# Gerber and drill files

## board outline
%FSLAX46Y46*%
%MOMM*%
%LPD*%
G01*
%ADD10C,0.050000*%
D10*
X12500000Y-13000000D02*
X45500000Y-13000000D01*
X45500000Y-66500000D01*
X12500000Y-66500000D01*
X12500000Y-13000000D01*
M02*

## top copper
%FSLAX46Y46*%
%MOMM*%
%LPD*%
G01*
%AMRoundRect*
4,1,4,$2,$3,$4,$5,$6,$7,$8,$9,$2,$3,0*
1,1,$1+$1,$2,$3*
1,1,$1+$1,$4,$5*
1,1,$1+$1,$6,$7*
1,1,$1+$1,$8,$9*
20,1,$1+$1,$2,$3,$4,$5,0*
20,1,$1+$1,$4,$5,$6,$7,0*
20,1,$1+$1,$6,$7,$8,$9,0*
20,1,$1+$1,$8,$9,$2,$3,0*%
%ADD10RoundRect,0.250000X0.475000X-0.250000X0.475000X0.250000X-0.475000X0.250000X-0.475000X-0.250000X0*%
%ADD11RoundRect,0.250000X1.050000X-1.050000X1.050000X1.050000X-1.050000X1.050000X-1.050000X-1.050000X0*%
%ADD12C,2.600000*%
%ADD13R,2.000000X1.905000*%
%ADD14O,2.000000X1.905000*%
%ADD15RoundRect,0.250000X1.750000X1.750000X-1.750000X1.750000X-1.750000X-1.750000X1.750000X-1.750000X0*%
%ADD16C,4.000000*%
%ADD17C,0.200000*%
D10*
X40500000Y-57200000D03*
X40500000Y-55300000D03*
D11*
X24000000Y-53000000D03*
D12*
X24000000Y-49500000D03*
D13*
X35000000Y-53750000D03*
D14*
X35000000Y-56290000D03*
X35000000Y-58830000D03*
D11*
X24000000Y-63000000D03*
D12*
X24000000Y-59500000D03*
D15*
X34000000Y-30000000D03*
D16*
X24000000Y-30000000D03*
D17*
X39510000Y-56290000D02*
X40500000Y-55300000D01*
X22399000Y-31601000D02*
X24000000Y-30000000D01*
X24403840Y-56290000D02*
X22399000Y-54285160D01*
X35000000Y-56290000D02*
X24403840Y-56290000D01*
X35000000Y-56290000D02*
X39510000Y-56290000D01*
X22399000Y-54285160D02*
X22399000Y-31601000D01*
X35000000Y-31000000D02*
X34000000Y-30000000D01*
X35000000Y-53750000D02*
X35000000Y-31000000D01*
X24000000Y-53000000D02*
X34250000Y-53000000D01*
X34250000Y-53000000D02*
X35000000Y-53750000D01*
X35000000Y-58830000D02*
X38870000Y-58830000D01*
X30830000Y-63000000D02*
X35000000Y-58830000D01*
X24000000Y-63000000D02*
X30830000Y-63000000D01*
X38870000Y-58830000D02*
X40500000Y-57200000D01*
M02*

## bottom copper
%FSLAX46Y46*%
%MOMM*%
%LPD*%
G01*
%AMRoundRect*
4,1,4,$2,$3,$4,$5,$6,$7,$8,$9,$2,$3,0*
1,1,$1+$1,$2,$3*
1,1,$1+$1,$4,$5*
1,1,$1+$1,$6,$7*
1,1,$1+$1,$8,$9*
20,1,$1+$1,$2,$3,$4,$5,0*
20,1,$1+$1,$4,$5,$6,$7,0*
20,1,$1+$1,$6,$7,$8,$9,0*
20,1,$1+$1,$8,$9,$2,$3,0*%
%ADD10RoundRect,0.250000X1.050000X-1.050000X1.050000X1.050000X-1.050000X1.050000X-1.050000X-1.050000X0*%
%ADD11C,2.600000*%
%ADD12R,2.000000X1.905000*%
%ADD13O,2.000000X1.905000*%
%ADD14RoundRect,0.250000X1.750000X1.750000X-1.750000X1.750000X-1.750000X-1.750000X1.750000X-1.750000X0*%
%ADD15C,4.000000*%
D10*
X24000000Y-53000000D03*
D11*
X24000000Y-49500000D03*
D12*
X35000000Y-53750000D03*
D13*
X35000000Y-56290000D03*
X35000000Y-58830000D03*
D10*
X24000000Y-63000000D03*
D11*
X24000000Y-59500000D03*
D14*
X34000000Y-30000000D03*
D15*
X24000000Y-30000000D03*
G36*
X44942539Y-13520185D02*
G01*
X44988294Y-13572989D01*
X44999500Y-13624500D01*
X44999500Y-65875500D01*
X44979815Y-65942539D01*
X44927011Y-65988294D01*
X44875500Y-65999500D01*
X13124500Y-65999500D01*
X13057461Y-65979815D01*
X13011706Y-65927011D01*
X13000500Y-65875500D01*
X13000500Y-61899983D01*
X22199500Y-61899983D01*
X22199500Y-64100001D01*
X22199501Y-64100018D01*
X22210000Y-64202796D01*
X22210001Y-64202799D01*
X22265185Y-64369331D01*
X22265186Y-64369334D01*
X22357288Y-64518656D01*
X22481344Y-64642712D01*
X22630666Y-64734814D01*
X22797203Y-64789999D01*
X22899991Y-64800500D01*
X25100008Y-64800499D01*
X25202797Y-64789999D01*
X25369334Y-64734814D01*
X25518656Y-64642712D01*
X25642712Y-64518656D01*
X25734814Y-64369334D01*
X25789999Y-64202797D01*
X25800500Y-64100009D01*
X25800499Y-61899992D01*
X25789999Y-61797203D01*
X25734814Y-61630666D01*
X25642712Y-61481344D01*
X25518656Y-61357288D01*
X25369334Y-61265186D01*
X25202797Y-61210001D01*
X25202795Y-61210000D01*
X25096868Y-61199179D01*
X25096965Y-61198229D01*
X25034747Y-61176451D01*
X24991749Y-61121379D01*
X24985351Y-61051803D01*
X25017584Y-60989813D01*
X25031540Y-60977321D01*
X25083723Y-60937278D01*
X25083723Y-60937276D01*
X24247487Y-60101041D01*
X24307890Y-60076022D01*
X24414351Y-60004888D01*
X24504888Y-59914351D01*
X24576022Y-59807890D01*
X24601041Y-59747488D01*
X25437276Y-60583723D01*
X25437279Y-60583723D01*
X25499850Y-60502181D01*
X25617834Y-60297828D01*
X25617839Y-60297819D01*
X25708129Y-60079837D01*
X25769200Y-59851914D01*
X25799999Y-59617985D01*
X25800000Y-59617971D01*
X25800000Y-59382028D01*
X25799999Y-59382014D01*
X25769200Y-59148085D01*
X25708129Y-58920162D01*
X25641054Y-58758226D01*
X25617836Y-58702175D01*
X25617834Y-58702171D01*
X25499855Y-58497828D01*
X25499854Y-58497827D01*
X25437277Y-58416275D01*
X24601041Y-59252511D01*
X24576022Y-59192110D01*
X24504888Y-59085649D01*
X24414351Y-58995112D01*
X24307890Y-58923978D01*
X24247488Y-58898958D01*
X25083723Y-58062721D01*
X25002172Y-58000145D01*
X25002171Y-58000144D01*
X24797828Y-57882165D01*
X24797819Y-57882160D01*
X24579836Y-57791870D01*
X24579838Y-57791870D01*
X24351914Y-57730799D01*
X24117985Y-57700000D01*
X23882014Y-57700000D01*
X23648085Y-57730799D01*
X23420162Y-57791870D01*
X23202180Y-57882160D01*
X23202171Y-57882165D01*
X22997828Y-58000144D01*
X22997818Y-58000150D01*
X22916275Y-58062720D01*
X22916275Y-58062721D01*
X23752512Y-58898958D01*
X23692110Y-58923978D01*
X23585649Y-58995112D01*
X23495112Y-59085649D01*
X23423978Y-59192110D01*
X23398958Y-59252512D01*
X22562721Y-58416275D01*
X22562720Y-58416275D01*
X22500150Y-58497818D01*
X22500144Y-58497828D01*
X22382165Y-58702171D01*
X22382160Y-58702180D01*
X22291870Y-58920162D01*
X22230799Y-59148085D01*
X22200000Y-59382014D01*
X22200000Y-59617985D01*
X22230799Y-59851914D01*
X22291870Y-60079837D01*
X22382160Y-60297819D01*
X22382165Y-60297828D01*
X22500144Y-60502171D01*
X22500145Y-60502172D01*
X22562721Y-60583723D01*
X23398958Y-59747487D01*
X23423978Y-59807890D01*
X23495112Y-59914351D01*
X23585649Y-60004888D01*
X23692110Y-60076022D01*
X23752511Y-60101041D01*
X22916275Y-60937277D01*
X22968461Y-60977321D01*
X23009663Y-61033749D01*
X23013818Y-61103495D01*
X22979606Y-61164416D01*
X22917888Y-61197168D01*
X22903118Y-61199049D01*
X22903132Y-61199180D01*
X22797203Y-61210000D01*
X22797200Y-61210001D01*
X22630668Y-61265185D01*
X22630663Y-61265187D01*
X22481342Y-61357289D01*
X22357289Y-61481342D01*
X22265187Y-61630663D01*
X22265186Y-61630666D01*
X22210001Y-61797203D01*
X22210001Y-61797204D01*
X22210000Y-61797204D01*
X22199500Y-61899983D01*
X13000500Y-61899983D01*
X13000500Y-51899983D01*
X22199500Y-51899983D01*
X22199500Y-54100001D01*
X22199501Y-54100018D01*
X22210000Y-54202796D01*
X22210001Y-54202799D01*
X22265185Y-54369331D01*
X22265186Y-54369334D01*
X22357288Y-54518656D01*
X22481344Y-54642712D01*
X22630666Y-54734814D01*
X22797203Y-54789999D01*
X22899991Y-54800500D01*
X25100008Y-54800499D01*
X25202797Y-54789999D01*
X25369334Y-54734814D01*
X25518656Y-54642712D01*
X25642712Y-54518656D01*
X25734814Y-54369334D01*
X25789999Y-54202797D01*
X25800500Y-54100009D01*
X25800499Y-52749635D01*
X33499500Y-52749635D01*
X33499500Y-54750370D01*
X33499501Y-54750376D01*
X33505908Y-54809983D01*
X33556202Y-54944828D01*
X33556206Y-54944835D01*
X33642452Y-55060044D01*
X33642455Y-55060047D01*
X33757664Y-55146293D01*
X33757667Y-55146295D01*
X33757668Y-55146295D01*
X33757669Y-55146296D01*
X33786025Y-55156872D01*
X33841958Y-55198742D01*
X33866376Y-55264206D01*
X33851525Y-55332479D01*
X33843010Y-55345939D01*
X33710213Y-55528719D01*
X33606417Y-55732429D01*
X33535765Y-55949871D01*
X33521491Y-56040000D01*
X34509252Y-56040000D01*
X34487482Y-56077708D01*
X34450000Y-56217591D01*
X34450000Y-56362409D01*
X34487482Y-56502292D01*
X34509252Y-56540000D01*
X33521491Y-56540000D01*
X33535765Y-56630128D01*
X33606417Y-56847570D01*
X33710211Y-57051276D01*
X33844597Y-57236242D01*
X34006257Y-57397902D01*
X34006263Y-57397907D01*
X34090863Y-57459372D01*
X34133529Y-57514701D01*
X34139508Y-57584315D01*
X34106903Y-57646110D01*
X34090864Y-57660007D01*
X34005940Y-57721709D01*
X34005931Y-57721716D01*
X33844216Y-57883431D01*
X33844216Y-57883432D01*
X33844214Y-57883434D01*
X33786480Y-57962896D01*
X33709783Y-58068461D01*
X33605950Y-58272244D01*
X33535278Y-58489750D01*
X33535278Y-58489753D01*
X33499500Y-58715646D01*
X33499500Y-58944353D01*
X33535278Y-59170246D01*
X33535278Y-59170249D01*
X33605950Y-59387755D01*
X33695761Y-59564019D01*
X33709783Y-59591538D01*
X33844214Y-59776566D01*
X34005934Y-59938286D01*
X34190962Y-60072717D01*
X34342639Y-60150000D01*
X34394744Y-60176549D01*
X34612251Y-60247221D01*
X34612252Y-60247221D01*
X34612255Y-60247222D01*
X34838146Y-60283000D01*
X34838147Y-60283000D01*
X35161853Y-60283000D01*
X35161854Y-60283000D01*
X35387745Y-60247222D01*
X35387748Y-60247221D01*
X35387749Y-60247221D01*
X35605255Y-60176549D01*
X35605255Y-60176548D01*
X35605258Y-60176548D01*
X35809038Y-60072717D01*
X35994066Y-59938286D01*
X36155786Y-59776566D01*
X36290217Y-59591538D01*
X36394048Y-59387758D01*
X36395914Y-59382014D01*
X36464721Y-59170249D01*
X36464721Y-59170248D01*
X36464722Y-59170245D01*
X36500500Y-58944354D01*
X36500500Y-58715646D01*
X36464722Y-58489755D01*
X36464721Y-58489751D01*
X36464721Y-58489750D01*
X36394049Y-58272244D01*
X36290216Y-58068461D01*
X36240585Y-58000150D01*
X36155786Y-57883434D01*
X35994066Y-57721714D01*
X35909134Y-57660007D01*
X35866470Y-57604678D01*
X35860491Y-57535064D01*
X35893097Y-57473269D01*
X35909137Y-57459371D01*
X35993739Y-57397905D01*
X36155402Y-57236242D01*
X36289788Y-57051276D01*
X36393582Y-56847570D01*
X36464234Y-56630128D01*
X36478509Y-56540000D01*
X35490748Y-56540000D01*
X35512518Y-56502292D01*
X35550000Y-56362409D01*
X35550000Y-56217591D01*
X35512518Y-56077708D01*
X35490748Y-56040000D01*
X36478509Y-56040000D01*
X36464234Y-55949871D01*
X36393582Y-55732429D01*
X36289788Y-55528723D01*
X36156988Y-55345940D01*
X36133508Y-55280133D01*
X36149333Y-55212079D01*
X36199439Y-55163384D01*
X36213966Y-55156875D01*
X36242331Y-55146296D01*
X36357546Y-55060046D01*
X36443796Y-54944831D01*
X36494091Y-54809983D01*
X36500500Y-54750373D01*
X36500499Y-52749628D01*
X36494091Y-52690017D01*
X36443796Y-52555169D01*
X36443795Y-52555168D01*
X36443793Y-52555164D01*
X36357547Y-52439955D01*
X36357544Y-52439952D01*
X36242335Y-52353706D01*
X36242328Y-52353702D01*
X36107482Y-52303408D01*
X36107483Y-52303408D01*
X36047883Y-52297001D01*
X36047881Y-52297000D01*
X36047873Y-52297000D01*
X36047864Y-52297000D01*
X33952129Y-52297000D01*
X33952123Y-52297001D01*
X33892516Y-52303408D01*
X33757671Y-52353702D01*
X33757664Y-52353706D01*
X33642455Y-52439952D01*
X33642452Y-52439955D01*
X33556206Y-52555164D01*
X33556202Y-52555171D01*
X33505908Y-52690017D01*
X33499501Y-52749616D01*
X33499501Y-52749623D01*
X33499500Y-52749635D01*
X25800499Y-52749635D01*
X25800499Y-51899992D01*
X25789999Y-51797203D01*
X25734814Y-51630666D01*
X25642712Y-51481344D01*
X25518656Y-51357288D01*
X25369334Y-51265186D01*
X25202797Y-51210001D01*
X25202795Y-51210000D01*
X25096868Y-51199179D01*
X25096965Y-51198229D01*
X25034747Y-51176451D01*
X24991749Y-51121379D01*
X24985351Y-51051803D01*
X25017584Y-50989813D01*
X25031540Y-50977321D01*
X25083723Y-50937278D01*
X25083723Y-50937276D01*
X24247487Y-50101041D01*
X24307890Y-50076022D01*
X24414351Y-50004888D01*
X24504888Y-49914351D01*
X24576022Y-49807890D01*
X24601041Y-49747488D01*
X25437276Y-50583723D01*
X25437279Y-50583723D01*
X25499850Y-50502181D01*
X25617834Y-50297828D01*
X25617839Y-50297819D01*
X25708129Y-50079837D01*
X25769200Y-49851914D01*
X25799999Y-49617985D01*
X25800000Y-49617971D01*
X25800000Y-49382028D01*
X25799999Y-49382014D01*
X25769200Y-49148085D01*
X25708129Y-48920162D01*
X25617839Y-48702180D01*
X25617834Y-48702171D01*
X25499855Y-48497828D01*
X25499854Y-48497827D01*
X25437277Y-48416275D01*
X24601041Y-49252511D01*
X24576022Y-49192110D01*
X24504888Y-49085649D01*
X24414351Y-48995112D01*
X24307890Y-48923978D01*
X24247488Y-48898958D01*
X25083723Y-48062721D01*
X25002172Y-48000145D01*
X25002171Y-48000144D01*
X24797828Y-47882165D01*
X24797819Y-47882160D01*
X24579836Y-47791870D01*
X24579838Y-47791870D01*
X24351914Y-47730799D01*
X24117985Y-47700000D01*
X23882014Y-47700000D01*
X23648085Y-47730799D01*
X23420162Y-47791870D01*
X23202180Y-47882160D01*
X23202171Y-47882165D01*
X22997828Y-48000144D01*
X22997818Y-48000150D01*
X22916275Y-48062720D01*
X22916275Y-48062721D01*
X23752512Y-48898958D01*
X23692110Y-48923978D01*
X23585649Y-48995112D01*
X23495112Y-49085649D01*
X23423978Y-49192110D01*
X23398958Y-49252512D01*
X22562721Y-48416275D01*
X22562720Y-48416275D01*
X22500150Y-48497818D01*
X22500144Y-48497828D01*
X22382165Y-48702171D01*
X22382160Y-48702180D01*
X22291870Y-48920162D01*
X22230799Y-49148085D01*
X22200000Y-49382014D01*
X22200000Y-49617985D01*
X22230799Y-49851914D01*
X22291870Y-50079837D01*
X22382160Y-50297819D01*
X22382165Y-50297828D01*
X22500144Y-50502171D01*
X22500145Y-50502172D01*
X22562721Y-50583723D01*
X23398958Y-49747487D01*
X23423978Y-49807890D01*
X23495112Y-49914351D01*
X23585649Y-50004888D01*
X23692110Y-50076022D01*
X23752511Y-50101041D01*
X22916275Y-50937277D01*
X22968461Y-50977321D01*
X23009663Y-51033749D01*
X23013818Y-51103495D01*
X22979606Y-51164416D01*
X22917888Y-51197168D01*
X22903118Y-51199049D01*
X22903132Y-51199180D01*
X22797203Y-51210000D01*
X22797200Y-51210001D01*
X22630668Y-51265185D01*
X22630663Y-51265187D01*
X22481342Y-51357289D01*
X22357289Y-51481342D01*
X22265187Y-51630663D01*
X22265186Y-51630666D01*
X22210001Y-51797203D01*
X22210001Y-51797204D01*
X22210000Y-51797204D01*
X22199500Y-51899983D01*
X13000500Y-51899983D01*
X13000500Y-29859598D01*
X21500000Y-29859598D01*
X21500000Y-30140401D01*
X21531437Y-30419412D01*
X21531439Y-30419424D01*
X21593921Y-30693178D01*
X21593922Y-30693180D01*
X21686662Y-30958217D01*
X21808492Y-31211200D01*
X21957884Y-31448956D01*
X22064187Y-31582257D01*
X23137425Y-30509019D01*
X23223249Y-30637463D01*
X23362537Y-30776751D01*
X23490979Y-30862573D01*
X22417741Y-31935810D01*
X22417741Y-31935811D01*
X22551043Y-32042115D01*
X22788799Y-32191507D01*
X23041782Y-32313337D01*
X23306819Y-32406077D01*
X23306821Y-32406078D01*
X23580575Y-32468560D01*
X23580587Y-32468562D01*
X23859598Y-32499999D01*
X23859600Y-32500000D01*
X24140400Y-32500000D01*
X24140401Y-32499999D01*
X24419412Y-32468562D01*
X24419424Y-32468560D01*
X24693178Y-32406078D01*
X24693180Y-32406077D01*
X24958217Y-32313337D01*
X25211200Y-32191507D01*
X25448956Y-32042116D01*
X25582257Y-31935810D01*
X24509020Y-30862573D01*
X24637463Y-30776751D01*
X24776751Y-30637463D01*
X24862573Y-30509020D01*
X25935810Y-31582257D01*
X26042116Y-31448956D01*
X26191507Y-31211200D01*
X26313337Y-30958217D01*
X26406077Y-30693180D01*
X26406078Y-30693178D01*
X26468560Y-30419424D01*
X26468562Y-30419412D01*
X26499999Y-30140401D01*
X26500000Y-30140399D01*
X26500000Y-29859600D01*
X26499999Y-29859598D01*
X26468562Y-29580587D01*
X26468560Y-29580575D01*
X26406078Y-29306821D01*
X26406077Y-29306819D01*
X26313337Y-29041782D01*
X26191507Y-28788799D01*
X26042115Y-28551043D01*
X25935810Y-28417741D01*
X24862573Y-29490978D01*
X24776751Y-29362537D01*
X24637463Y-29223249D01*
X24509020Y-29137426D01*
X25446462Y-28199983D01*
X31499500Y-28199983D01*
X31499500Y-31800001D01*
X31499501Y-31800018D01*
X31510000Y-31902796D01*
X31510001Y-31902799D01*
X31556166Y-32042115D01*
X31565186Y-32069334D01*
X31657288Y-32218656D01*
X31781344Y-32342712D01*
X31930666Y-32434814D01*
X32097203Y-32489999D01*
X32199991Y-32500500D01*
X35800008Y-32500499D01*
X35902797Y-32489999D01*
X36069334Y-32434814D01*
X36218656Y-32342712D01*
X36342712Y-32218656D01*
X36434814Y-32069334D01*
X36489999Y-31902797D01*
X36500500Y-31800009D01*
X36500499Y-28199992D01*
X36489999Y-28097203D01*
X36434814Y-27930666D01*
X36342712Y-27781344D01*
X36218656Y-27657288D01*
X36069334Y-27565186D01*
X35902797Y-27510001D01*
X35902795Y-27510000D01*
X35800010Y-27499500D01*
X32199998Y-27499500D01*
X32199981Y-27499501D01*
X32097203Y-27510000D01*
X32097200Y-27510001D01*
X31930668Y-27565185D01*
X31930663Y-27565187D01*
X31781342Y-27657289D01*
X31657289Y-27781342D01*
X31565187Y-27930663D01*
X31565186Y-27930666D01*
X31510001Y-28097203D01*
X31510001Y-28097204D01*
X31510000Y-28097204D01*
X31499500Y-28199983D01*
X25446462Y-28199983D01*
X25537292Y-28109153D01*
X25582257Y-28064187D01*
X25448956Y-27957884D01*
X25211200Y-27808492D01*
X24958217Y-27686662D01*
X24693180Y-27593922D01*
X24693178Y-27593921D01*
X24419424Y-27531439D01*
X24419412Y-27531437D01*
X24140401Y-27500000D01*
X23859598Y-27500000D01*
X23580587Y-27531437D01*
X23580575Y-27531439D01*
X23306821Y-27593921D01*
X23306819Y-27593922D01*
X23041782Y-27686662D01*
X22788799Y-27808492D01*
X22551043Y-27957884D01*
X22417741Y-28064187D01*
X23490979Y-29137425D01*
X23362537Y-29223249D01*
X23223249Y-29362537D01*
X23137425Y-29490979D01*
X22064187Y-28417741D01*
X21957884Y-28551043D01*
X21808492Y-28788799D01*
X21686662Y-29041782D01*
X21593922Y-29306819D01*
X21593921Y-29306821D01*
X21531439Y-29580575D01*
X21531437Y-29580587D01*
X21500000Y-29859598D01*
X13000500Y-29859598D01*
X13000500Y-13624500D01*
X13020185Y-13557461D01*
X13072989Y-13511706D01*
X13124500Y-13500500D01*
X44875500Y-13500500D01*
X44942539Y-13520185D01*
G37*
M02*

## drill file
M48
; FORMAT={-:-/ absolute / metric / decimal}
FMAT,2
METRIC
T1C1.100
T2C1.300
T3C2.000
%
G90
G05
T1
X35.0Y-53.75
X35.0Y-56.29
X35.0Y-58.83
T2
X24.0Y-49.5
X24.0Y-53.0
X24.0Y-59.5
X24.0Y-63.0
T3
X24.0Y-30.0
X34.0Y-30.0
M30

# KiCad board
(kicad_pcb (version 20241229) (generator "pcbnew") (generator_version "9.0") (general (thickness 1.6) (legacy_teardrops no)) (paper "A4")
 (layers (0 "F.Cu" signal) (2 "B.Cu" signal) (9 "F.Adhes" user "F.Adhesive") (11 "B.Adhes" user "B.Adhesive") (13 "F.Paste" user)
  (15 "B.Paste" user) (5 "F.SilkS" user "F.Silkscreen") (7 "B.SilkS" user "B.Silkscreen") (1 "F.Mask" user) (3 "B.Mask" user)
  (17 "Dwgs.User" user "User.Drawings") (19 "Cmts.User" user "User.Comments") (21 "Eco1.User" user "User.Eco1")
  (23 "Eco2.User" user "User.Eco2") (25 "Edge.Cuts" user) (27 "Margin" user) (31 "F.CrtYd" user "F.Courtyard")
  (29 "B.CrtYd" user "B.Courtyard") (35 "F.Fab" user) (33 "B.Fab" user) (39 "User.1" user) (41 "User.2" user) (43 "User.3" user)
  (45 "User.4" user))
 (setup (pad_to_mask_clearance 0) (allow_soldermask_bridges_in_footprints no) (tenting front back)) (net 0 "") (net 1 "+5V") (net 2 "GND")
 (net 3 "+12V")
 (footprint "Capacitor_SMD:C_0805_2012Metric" (layer "F.Cu") (at 40.5 56.25 90)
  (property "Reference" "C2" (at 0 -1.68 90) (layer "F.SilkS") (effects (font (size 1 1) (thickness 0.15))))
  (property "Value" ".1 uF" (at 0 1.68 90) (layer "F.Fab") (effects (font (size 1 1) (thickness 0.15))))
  (pad "1" smd roundrect (at -0.95 0 90) (size 1 1.45) (layers "F.Cu" "F.Mask" "F.Paste") (roundrect_rratio 0.25) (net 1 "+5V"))
  (pad "2" smd roundrect (at 0.95 0 90) (size 1 1.45) (layers "F.Cu" "F.Mask" "F.Paste") (roundrect_rratio 0.25) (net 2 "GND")))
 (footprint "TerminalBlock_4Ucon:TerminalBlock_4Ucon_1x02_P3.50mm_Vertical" (layer "F.Cu") (at 24 53 90)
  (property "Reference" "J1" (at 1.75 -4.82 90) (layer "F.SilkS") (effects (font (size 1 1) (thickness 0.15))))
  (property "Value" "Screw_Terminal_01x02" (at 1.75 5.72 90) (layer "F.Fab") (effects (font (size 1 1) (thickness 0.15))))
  (pad "1" thru_hole roundrect (at 0 0 90) (size 2.6 2.6) (drill 1.3) (layers "*.Cu" "*.Mask") (remove_unused_layers no)
   (roundrect_rratio 0.096154) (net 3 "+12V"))
  (pad "2" thru_hole circle (at 3.5 0 90) (size 2.6 2.6) (drill 1.3) (layers "*.Cu" "*.Mask") (remove_unused_layers no) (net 2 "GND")))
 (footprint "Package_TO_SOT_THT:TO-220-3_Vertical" (layer "F.Cu") (at 35 53.75 -90)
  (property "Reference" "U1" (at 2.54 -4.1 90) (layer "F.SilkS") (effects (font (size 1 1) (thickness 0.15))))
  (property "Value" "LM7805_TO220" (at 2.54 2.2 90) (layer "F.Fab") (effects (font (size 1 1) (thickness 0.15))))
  (pad "1" thru_hole rect (at 0 0 270) (size 1.905 2) (drill 1.1) (layers "*.Cu" "*.Mask") (remove_unused_layers no) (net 3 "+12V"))
  (pad "2" thru_hole oval (at 2.54 0 270) (size 1.905 2) (drill 1.1) (layers "*.Cu" "*.Mask") (remove_unused_layers no) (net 2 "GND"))
  (pad "3" thru_hole oval (at 5.08 0 270) (size 1.905 2) (drill 1.1) (layers "*.Cu" "*.Mask") (remove_unused_layers no) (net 1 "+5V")))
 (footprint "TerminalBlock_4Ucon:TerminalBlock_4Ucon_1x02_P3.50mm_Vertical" (layer "F.Cu") (at 24 63 90)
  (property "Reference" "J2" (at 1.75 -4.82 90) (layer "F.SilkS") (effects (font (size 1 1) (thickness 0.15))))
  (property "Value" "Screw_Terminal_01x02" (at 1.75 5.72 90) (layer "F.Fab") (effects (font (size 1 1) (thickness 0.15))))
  (pad "1" thru_hole roundrect (at 0 0 90) (size 2.6 2.6) (drill 1.3) (layers "*.Cu" "*.Mask") (remove_unused_layers no)
   (roundrect_rratio 0.096154) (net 1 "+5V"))
  (pad "2" thru_hole circle (at 3.5 0 90) (size 2.6 2.6) (drill 1.3) (layers "*.Cu" "*.Mask") (remove_unused_layers no) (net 2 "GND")))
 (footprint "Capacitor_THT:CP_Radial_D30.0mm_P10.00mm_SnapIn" (layer "F.Cu") (at 34 30 180)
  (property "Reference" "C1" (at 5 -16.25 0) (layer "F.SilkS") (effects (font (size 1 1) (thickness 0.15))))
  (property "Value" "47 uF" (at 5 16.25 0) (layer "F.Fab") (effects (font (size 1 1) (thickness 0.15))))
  (pad "1" thru_hole roundrect (at 0 0 180) (size 4 4) (drill 2) (layers "*.Cu" "*.Mask") (remove_unused_layers no)
   (roundrect_rratio 0.0625) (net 3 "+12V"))
  (pad "2" thru_hole circle (at 10 0 180) (size 4 4) (drill 2) (layers "*.Cu" "*.Mask") (remove_unused_layers no) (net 2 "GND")))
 (gr_rect (start 12.5 13) (end 45.5 66.5) (stroke (width 0.05) (type default)) (fill no) (layer "Edge.Cuts"))
 (segment (start 39.51 56.29) (end 40.5 55.3) (width 0.2) (layer "F.Cu") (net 2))
 (segment (start 22.399 31.601) (end 24 30) (width 0.2) (layer "F.Cu") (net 2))
 (segment (start 24.40384 56.29) (end 22.399 54.28516) (width 0.2) (layer "F.Cu") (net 2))
 (segment (start 35 56.29) (end 24.40384 56.29) (width 0.2) (layer "F.Cu") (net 2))
 (segment (start 35 56.29) (end 39.51 56.29) (width 0.2) (layer "F.Cu") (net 2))
 (segment (start 22.399 54.28516) (end 22.399 31.601) (width 0.2) (layer "F.Cu") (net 2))
 (segment (start 35 31) (end 34 30) (width 0.2) (layer "F.Cu") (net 3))
 (segment (start 35 53.75) (end 35 31) (width 0.2) (layer "F.Cu") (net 3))
 (segment (start 24 53) (end 34.25 53) (width 0.2) (layer "F.Cu") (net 3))
 (segment (start 34.25 53) (end 35 53.75) (width 0.2) (layer "F.Cu") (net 3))
 (segment (start 35 58.83) (end 38.87 58.83) (width 0.2) (layer "F.Cu") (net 1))
 (segment (start 30.83 63) (end 35 58.83) (width 0.2) (layer "F.Cu") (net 1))
 (segment (start 24 63) (end 30.83 63) (width 0.2) (layer "F.Cu") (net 1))
 (segment (start 38.87 58.83) (end 40.5 57.2) (width 0.2) (layer "F.Cu") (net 1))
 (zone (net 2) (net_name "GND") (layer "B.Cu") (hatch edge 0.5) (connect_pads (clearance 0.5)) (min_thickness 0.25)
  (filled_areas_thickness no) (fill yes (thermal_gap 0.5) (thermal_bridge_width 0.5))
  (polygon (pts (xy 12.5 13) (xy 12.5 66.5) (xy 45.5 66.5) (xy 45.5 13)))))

